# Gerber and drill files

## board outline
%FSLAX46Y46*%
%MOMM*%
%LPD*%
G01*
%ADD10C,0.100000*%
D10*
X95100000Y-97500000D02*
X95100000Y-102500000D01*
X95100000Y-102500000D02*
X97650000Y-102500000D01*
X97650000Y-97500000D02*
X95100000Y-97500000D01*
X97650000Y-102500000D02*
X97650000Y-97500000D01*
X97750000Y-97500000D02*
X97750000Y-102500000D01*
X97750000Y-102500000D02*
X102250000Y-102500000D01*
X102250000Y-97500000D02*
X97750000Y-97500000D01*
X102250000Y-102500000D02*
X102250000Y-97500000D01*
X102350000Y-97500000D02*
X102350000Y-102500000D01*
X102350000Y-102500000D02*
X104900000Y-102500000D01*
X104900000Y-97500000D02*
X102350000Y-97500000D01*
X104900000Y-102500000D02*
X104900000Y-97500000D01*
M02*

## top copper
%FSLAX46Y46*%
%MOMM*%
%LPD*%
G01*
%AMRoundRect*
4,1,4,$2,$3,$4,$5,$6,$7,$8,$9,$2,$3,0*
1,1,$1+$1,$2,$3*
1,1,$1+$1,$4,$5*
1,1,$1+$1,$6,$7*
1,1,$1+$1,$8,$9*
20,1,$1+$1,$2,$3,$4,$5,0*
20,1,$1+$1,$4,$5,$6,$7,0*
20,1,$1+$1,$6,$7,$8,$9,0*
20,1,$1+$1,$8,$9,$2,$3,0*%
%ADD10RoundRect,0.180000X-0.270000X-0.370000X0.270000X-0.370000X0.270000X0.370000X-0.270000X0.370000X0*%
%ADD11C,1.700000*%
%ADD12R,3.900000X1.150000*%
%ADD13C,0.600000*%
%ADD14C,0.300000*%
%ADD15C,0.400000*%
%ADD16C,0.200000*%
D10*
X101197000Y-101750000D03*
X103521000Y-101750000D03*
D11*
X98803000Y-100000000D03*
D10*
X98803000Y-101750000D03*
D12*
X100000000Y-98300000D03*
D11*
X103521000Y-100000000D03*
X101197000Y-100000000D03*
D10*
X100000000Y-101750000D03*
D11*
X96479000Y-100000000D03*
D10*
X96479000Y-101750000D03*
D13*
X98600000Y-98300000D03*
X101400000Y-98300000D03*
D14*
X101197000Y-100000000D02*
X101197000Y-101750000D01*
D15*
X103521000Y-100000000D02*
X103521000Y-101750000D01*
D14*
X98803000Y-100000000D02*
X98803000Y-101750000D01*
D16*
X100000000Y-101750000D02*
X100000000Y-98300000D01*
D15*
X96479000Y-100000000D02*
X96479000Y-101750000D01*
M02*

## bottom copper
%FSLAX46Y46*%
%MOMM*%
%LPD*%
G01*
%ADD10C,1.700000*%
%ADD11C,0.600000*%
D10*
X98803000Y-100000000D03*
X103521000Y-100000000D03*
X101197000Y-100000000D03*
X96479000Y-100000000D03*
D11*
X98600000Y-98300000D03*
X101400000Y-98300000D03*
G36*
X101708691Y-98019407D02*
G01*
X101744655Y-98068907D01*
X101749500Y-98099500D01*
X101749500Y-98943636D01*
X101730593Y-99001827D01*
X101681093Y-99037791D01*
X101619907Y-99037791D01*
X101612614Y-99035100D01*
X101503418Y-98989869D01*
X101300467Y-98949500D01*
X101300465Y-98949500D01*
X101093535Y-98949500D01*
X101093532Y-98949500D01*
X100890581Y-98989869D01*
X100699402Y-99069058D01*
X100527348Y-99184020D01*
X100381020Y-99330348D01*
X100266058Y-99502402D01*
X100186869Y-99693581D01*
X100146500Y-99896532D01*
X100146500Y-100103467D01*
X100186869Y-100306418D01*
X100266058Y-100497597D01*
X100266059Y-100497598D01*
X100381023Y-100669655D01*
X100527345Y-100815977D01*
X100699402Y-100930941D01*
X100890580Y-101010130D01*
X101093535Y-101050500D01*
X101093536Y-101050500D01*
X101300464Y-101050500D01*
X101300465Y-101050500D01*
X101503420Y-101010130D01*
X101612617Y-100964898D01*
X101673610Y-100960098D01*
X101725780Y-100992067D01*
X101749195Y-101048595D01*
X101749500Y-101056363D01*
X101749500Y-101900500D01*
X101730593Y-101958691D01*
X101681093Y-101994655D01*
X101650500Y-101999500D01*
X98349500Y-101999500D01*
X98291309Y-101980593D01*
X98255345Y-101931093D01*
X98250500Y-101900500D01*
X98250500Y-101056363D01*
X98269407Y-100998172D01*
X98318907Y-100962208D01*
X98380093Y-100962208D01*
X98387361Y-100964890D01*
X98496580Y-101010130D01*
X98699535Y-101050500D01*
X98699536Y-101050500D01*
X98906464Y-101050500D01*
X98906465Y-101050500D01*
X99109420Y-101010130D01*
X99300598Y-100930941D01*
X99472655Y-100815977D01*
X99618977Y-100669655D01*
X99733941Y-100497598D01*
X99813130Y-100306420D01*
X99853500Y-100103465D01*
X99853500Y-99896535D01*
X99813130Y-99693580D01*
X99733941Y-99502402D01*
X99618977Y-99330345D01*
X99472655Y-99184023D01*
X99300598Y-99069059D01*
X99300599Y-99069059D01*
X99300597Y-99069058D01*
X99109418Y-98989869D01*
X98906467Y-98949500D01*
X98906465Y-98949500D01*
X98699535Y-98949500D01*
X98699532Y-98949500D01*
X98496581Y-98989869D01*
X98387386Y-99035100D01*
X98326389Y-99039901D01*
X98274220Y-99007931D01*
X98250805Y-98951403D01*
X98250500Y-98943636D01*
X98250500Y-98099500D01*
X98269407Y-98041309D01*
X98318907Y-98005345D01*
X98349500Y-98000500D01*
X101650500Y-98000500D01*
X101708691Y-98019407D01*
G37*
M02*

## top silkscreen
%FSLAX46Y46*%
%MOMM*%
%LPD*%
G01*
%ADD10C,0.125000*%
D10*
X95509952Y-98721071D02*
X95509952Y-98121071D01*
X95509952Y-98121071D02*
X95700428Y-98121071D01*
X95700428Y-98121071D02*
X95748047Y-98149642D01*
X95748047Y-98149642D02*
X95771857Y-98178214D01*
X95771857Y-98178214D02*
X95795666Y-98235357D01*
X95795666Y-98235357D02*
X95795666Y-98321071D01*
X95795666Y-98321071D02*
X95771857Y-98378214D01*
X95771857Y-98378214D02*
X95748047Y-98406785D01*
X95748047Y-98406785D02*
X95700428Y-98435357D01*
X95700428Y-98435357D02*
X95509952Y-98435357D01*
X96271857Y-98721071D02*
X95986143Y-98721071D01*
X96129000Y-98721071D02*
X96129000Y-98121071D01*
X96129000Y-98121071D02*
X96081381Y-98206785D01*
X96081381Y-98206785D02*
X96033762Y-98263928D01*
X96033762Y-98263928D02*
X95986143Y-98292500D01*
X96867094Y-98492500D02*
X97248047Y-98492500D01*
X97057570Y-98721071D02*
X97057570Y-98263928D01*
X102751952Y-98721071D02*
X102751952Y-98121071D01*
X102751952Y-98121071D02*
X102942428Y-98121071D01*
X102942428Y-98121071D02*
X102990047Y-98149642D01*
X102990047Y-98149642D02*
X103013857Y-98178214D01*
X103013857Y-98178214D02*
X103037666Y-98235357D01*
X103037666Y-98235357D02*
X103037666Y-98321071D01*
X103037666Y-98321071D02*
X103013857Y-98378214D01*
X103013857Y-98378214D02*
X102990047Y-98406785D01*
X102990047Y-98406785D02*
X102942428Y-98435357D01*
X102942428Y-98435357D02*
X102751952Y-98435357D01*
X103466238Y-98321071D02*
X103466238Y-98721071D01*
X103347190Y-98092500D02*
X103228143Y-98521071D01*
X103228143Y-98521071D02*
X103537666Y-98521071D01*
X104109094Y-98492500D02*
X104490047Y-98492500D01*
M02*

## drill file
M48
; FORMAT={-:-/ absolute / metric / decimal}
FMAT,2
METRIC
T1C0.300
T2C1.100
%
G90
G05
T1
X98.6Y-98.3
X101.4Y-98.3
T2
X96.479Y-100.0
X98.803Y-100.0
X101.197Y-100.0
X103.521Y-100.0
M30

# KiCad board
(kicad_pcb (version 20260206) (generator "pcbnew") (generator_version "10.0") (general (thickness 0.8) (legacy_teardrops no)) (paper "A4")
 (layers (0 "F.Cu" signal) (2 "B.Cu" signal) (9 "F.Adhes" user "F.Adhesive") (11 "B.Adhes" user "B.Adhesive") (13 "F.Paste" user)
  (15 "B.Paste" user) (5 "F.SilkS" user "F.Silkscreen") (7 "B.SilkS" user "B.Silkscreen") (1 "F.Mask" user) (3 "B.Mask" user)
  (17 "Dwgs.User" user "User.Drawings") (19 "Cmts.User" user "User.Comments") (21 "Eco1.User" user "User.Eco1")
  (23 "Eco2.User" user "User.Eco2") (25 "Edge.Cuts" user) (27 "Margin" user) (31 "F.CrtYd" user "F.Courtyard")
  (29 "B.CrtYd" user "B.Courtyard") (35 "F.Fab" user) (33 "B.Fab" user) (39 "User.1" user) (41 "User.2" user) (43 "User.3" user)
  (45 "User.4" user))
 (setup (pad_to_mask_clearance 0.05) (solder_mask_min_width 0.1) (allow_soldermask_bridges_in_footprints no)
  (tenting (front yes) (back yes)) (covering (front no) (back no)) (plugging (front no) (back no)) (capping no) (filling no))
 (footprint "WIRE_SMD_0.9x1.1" (layer "F.Cu") (at 101.197 101.75)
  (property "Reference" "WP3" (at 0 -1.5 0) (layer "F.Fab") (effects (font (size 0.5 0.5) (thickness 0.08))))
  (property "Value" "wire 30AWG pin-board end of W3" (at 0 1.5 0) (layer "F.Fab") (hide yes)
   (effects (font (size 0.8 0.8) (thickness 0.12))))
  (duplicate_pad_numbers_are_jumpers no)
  (pad "1" smd roundrect (at 0 0) (size 0.9 1.1) (layers "F.Cu" "F.Mask") (roundrect_rratio 0.2) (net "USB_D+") (thermal_bridge_angle 45)))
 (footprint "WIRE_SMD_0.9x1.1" (layer "F.Cu") (at 103.521 101.75)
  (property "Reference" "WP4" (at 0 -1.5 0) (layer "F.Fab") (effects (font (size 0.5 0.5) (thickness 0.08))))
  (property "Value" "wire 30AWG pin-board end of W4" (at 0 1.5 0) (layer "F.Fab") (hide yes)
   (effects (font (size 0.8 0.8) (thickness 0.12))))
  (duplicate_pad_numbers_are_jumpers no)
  (pad "1" smd roundrect (at 0 0) (size 0.9 1.1) (layers "F.Cu" "F.Mask") (roundrect_rratio 0.2) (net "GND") (thermal_bridge_angle 45)))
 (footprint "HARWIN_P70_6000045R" (layer "F.Cu") (at 98.803 100)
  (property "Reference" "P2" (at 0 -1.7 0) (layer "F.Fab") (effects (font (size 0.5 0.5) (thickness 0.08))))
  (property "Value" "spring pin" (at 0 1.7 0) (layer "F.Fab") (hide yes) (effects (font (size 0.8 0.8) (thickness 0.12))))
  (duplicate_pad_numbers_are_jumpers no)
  (pad "1" thru_hole circle (at 0 0) (size 1.7 1.7) (drill 1.1) (layers "*.Cu" "*.Mask") (remove_unused_layers no) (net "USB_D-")))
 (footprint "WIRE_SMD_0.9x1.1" (layer "F.Cu") (at 98.803 101.75)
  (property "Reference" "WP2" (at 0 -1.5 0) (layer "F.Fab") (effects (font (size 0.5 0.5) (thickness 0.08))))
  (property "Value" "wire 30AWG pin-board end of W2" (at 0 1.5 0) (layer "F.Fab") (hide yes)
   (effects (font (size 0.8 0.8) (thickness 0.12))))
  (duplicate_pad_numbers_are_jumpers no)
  (pad "1" smd roundrect (at 0 0) (size 0.9 1.1) (layers "F.Cu" "F.Mask") (roundrect_rratio 0.2) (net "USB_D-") (thermal_bridge_angle 45)))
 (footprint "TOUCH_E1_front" (layer "F.Cu") (at 100 98.3)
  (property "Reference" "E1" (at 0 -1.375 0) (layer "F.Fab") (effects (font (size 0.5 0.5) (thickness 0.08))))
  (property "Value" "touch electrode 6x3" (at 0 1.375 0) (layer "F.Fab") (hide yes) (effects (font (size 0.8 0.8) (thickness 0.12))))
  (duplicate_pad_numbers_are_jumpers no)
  (pad "1" smd rect (at 0 0) (size 3.9 1.15) (layers "F.Cu" "F.Mask") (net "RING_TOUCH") (thermal_bridge_angle 45)))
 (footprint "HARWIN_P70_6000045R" (layer "F.Cu") (at 103.521 100)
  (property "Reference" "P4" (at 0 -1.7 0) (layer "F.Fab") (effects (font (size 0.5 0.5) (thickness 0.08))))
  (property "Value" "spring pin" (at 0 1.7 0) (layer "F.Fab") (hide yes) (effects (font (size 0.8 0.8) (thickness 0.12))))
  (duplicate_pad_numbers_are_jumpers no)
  (pad "1" thru_hole circle (at 0 0) (size 1.7 1.7) (drill 1.1) (layers "*.Cu" "*.Mask") (remove_unused_layers no) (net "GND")))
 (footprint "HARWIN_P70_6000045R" (layer "F.Cu") (at 101.197 100)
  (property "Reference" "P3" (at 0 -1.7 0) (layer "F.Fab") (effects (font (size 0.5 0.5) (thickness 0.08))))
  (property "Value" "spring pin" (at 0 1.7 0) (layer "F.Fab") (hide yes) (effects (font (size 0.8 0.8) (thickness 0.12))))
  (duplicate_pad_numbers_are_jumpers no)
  (pad "1" thru_hole circle (at 0 0) (size 1.7 1.7) (drill 1.1) (layers "*.Cu" "*.Mask") (remove_unused_layers no) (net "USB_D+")))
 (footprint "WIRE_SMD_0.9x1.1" (layer "F.Cu") (at 100 101.75)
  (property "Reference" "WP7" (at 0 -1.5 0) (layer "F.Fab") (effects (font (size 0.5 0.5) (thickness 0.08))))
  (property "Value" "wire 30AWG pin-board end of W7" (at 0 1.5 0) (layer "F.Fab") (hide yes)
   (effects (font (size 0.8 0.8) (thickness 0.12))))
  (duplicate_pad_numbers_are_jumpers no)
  (pad "1" smd roundrect (at 0 0) (size 0.9 1.1) (layers "F.Cu" "F.Mask") (roundrect_rratio 0.2) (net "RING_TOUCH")
   (thermal_bridge_angle 45)))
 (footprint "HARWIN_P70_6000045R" (layer "F.Cu") (at 96.479 100)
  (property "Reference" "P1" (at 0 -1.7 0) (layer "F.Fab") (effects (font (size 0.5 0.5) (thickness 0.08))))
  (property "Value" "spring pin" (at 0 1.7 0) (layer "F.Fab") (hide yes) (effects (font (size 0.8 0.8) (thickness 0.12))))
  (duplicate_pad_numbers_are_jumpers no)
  (pad "1" thru_hole circle (at 0 0) (size 1.7 1.7) (drill 1.1) (layers "*.Cu" "*.Mask") (remove_unused_layers no) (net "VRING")))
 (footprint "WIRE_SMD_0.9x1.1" (layer "F.Cu") (at 96.479 101.75)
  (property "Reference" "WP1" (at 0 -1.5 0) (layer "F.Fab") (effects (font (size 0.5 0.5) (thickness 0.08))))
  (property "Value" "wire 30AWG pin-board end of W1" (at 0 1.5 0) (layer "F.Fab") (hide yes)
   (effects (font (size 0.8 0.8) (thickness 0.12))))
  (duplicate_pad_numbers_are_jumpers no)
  (pad "1" smd roundrect (at 0 0) (size 0.9 1.1) (layers "F.Cu" "F.Mask") (roundrect_rratio 0.2) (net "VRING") (thermal_bridge_angle 45)))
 (gr_line (start 95.1 97.5) (end 95.1 102.5) (stroke (width 0.1) (type default)) (layer "Edge.Cuts"))
 (gr_line (start 95.1 102.5) (end 97.65 102.5) (stroke (width 0.1) (type default)) (layer "Edge.Cuts"))
 (gr_line (start 97.65 97.5) (end 95.1 97.5) (stroke (width 0.1) (type default)) (layer "Edge.Cuts"))
 (gr_line (start 97.65 102.5) (end 97.65 97.5) (stroke (width 0.1) (type default)) (layer "Edge.Cuts"))
 (gr_line (start 97.75 97.5) (end 97.75 102.5) (stroke (width 0.1) (type default)) (layer "Edge.Cuts"))
 (gr_line (start 97.75 102.5) (end 102.25 102.5) (stroke (width 0.1) (type default)) (layer "Edge.Cuts"))
 (gr_line (start 102.25 97.5) (end 97.75 97.5) (stroke (width 0.1) (type default)) (layer "Edge.Cuts"))
 (gr_line (start 102.25 102.5) (end 102.25 97.5) (stroke (width 0.1) (type default)) (layer "Edge.Cuts"))
 (gr_line (start 102.35 97.5) (end 102.35 102.5) (stroke (width 0.1) (type default)) (layer "Edge.Cuts"))
 (gr_line (start 102.35 102.5) (end 104.9 102.5) (stroke (width 0.1) (type default)) (layer "Edge.Cuts"))
 (gr_line (start 104.9 97.5) (end 102.35 97.5) (stroke (width 0.1) (type default)) (layer "Edge.Cuts"))
 (gr_line (start 104.9 102.5) (end 104.9 97.5) (stroke (width 0.1) (type default)) (layer "Edge.Cuts"))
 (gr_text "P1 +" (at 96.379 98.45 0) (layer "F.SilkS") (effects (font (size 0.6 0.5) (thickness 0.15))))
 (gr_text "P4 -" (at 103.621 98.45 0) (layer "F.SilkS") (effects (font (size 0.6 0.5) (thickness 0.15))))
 (segment (start 101.197 100) (end 101.197 101.75) (width 0.3) (layer "F.Cu") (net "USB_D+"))
 (segment (start 103.521 100) (end 103.521 101.75) (width 0.4) (layer "F.Cu") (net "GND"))
 (segment (start 98.803 100) (end 98.803 101.75) (width 0.3) (layer "F.Cu") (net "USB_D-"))
 (segment (start 100 101.75) (end 100 98.3) (width 0.2) (layer "F.Cu") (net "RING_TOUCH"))
 (via (at 98.6 98.3) (size 0.6) (drill 0.3) (layers "F.Cu" "B.Cu") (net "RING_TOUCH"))
 (via (at 101.4 98.3) (size 0.6) (drill 0.3) (layers "F.Cu" "B.Cu") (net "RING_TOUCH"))
 (segment (start 96.479 100) (end 96.479 101.75) (width 0.4) (layer "F.Cu") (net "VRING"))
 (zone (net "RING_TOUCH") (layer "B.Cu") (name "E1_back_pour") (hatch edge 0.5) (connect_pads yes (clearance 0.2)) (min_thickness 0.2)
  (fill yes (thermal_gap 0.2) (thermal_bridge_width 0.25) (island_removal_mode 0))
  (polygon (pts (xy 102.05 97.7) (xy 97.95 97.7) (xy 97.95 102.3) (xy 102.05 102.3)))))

